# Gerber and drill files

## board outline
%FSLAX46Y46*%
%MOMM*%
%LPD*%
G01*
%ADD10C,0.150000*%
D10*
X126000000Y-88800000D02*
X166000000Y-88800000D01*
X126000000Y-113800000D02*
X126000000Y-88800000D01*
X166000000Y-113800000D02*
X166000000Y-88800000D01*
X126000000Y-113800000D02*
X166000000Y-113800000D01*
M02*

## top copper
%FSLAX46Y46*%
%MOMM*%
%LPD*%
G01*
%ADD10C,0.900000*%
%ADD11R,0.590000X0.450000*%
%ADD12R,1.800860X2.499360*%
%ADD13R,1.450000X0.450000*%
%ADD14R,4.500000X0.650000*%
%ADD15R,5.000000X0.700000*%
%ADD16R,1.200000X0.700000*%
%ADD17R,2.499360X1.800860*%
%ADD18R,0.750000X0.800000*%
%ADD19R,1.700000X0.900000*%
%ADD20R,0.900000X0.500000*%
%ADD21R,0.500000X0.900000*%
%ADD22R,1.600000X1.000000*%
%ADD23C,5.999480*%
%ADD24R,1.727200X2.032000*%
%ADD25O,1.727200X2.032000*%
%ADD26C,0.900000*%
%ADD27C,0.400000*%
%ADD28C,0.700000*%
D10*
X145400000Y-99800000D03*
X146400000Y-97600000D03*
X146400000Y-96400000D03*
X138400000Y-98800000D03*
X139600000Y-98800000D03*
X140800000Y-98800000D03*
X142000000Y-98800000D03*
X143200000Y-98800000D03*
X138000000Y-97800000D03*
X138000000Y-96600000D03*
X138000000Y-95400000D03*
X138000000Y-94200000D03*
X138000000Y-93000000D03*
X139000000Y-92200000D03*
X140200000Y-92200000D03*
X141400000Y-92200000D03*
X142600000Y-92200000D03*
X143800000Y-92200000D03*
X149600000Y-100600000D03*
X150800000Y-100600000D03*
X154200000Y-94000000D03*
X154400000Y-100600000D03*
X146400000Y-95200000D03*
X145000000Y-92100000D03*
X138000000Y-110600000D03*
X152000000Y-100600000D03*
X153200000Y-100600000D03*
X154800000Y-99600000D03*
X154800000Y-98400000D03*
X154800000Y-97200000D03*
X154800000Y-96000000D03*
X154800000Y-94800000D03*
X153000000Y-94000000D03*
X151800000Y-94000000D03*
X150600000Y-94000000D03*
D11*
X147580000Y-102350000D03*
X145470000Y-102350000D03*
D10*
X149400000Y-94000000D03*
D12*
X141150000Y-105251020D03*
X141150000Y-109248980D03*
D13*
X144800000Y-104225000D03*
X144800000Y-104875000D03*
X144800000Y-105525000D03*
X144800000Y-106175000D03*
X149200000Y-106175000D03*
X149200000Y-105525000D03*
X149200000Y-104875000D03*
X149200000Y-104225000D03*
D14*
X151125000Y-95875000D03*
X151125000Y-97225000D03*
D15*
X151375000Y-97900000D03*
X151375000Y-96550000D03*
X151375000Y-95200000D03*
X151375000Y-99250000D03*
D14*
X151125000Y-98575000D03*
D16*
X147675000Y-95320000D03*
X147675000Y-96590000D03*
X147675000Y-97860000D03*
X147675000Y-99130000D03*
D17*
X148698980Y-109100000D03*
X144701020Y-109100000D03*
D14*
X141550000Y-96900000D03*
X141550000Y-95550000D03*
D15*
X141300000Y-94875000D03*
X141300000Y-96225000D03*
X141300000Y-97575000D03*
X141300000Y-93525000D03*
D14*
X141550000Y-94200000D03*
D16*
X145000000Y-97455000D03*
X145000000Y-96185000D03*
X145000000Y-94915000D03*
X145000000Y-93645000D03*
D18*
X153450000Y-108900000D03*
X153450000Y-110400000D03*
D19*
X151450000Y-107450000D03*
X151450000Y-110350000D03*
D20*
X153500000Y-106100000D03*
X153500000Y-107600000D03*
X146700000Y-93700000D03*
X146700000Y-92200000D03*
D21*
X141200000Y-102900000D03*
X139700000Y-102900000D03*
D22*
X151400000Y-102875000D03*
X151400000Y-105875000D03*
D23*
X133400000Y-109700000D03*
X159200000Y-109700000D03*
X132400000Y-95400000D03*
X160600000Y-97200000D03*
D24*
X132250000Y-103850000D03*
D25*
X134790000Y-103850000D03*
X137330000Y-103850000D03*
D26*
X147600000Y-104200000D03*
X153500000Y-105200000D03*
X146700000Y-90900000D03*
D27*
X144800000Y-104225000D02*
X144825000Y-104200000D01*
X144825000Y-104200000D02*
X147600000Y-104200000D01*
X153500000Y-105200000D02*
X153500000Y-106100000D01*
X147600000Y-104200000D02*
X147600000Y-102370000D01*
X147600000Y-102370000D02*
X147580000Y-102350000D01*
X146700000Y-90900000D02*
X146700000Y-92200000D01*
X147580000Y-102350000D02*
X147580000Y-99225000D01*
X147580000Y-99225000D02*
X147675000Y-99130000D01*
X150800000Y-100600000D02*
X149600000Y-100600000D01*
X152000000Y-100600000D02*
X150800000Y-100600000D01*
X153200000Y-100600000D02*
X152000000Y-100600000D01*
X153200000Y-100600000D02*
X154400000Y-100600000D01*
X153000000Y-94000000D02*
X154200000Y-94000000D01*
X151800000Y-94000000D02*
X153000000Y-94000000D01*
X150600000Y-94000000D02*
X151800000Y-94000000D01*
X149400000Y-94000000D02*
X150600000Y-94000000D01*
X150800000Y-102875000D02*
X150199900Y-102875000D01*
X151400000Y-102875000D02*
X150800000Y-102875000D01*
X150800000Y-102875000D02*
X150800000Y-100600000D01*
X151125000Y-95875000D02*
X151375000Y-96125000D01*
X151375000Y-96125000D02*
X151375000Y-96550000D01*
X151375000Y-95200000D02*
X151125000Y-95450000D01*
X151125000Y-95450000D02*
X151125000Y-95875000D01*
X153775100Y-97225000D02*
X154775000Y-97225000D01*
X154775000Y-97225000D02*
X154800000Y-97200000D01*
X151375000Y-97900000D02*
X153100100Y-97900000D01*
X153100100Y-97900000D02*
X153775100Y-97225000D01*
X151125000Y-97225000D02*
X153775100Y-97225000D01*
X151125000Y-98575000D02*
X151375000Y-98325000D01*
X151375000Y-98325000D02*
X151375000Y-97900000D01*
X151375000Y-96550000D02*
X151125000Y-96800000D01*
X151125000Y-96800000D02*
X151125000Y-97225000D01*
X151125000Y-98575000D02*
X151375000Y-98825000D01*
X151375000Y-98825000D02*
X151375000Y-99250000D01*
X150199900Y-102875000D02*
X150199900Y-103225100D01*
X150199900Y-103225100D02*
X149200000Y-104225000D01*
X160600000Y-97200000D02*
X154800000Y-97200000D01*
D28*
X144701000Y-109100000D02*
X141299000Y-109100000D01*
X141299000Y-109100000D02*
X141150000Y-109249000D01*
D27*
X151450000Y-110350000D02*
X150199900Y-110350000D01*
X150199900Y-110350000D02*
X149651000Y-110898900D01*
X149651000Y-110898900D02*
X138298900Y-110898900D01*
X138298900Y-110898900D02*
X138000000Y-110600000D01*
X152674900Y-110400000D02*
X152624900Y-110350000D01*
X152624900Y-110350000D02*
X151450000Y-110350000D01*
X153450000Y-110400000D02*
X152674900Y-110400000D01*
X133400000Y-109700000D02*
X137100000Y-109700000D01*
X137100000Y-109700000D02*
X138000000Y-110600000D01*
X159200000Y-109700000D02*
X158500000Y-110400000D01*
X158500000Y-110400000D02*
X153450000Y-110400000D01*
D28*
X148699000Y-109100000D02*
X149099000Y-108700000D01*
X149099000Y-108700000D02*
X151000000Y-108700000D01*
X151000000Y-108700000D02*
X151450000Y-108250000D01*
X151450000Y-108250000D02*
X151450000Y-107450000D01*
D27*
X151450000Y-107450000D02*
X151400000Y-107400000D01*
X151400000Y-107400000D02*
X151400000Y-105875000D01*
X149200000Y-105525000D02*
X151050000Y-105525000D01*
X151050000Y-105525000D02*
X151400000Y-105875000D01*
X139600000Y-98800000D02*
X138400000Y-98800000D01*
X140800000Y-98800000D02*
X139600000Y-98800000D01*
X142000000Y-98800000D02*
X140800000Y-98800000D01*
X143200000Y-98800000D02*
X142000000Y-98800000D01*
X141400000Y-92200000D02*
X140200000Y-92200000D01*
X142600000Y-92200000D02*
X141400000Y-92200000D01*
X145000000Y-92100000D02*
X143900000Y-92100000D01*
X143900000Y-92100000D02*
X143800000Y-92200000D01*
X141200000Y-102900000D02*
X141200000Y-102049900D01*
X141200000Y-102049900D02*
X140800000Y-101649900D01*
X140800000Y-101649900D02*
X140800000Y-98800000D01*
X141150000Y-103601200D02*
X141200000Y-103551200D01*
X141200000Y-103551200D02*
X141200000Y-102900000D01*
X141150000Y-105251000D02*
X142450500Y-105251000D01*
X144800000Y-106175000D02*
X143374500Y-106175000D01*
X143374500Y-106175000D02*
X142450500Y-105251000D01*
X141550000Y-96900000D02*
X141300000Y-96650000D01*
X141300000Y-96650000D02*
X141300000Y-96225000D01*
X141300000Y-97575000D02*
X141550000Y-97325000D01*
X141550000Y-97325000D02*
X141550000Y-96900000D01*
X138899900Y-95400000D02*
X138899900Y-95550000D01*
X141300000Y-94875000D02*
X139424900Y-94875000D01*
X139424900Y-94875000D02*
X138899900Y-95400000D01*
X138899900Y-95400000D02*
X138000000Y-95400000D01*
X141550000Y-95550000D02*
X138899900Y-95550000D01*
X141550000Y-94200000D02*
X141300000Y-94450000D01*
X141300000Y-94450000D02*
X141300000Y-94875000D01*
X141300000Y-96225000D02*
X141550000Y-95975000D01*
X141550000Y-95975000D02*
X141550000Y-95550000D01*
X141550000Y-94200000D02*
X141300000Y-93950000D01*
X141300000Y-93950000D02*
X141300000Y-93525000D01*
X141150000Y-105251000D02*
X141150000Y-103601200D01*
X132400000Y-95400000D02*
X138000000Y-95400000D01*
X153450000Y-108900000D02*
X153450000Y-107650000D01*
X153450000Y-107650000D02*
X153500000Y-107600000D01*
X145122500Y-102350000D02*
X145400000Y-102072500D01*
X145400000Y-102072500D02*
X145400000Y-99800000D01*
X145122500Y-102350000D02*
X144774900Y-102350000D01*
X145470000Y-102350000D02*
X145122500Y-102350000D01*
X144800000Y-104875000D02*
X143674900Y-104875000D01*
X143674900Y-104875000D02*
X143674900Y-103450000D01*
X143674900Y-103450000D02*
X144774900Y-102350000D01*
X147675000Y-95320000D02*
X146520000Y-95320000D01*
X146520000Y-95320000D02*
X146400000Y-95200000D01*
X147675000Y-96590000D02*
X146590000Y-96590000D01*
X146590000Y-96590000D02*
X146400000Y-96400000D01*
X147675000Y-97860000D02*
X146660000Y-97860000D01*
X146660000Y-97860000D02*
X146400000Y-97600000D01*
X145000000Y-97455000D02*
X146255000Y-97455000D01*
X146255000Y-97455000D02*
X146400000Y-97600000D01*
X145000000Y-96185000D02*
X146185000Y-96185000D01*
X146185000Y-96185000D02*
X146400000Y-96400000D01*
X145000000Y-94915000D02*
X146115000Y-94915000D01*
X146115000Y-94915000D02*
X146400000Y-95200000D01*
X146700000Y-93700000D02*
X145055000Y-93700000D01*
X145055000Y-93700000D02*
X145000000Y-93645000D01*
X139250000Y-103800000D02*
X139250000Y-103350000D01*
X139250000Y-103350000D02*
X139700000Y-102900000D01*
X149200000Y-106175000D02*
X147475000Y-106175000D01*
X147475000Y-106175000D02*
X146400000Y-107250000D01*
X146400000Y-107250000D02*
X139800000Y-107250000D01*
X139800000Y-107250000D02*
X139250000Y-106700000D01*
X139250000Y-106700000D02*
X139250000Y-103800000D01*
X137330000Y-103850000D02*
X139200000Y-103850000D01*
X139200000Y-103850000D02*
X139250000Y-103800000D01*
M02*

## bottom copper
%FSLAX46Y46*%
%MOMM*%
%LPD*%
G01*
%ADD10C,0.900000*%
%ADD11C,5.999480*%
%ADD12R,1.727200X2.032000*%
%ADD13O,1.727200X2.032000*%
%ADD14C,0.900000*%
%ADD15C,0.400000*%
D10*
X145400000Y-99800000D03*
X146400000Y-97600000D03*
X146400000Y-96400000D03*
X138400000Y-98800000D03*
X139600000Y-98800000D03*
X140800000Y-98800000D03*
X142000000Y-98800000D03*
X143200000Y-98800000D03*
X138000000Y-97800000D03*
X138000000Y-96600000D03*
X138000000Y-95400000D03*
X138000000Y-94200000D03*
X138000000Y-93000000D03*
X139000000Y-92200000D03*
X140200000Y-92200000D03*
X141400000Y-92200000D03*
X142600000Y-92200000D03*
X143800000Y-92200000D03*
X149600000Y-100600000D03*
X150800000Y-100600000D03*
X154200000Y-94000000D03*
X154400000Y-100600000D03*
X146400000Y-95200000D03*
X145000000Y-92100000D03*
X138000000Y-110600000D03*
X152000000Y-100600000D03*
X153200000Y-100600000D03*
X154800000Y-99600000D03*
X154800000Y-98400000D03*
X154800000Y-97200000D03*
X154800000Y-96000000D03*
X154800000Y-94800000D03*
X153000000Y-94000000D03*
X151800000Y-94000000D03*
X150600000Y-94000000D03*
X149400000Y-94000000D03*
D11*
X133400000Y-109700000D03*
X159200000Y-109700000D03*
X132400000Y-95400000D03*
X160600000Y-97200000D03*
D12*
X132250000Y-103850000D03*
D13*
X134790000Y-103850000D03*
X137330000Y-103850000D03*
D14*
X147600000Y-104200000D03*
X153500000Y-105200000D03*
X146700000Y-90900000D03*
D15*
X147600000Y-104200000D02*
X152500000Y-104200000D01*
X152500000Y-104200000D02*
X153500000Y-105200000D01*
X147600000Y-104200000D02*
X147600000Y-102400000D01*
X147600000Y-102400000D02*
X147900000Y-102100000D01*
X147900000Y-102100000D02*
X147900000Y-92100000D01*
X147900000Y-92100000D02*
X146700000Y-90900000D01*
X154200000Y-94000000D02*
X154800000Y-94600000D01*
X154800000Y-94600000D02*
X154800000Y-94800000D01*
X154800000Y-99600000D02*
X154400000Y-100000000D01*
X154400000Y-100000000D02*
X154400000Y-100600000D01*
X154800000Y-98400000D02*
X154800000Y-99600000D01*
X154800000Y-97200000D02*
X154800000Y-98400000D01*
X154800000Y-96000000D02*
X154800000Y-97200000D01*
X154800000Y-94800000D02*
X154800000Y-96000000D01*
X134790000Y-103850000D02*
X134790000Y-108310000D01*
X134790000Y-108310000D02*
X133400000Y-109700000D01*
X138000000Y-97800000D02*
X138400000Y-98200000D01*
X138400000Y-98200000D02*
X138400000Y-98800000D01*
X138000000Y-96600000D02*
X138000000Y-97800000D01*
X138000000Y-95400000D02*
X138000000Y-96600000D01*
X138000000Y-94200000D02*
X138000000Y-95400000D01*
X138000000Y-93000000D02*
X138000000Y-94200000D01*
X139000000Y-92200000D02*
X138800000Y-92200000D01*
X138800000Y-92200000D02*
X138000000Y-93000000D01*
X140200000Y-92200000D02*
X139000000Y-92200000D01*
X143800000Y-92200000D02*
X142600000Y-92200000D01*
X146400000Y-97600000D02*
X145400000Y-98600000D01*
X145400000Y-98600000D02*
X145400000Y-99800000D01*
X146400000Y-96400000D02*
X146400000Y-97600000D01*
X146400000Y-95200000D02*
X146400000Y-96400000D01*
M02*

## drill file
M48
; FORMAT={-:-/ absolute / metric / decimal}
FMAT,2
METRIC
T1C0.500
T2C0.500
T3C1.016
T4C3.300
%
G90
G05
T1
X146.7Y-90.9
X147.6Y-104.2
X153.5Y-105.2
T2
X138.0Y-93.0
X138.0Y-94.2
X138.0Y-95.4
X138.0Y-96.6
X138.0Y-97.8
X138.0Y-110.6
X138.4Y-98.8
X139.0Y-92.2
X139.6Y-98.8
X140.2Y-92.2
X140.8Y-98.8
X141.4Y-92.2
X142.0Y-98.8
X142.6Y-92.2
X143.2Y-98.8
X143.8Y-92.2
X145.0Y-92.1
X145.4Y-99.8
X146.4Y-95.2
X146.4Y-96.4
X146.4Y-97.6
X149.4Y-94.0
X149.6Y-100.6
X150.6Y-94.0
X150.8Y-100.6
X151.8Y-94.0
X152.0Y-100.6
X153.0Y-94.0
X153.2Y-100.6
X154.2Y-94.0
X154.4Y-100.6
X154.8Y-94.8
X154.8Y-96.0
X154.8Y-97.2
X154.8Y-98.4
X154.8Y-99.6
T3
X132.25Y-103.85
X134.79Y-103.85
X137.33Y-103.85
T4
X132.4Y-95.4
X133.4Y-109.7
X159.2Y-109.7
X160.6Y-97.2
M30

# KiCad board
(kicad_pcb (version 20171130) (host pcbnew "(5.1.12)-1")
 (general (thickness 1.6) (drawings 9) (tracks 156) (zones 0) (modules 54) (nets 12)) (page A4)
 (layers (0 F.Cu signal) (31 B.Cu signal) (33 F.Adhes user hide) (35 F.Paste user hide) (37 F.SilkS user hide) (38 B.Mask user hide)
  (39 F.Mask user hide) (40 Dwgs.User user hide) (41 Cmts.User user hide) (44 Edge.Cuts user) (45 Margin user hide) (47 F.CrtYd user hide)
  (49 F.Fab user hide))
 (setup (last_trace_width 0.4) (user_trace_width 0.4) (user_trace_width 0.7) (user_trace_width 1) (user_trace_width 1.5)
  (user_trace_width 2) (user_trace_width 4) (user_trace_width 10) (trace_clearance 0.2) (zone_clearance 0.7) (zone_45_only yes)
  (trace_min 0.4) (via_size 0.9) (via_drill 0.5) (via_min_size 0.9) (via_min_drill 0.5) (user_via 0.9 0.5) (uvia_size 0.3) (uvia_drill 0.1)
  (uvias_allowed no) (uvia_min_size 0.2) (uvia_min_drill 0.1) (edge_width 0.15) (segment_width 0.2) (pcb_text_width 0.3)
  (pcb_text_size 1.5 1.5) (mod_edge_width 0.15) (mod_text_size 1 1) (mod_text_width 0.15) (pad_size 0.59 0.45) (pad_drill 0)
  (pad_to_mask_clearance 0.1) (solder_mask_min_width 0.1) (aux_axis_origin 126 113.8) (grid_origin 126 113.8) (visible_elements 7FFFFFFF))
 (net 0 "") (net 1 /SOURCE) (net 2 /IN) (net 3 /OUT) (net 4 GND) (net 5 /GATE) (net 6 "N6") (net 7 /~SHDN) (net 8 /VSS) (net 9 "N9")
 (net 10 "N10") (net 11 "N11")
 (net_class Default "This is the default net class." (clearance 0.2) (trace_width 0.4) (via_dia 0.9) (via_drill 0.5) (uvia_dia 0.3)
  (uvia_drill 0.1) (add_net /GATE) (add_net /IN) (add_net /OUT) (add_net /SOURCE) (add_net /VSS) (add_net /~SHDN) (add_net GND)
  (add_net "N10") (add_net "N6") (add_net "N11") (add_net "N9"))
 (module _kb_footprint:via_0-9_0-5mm (layer F.Cu) (at 145.4 99.8)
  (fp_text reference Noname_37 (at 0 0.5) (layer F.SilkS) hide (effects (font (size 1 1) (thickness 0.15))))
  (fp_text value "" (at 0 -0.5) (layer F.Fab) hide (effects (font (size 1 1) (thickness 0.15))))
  (pad 1 thru_hole circle (at 0 0) (size 0.9 0.9) (drill 0.5) (layers *.Cu) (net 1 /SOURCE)))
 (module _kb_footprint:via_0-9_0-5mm (layer F.Cu) (at 146.4 97.6)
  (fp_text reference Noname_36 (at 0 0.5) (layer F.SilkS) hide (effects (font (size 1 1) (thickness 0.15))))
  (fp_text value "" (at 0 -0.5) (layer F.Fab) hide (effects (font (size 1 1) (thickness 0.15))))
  (pad 1 thru_hole circle (at 0 0) (size 0.9 0.9) (drill 0.5) (layers *.Cu) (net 1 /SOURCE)))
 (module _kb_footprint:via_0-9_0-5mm (layer F.Cu) (at 146.4 96.4)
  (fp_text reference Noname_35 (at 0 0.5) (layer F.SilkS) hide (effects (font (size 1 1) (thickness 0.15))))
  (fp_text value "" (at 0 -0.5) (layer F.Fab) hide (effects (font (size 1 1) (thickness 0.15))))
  (pad 1 thru_hole circle (at 0 0) (size 0.9 0.9) (drill 0.5) (layers *.Cu) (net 1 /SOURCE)))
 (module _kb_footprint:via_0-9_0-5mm (layer F.Cu) (at 138.4 98.8)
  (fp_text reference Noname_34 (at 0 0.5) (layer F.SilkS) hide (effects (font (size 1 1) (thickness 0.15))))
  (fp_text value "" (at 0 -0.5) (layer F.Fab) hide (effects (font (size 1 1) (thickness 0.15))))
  (pad 1 thru_hole circle (at 0 0) (size 0.9 0.9) (drill 0.5) (layers *.Cu) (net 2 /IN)))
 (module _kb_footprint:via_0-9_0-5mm (layer F.Cu) (at 139.6 98.8)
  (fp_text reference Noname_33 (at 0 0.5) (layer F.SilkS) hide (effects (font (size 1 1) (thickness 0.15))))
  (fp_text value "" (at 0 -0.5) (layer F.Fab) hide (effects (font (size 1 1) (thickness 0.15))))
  (pad 1 thru_hole circle (at 0 0) (size 0.9 0.9) (drill 0.5) (layers *.Cu) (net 2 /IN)))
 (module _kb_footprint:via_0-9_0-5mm (layer F.Cu) (at 140.8 98.8)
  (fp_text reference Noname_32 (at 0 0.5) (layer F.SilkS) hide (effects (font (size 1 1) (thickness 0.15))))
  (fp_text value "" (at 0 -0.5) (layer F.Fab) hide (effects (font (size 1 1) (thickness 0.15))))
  (pad 1 thru_hole circle (at 0 0) (size 0.9 0.9) (drill 0.5) (layers *.Cu) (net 2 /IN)))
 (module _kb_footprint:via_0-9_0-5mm (layer F.Cu) (at 142 98.8)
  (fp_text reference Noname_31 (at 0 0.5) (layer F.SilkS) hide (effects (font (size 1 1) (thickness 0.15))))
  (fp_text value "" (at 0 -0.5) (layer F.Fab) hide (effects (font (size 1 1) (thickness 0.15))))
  (pad 1 thru_hole circle (at 0 0) (size 0.9 0.9) (drill 0.5) (layers *.Cu) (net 2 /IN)))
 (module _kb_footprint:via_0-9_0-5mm (layer F.Cu) (at 143.2 98.8)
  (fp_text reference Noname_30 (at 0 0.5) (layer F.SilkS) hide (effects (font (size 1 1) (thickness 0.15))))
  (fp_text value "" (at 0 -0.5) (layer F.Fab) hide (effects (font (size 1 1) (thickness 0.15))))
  (pad 1 thru_hole circle (at 0 0) (size 0.9 0.9) (drill 0.5) (layers *.Cu) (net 2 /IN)))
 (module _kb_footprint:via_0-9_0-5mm (layer F.Cu) (at 138 97.8)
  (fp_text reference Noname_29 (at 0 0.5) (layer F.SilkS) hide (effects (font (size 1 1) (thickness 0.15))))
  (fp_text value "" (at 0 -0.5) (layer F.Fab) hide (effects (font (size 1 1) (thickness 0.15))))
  (pad 1 thru_hole circle (at 0 0) (size 0.9 0.9) (drill 0.5) (layers *.Cu) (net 2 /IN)))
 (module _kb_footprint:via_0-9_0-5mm (layer F.Cu) (at 138 96.6)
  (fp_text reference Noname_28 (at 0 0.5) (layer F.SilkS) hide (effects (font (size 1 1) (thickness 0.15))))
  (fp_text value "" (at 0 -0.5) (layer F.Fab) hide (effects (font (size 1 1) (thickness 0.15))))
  (pad 1 thru_hole circle (at 0 0) (size 0.9 0.9) (drill 0.5) (layers *.Cu) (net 2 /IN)))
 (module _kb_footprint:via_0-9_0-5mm (layer F.Cu) (at 138 95.4)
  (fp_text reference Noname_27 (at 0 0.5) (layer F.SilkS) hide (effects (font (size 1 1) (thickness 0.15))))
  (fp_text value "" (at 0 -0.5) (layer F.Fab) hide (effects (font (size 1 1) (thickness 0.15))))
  (pad 1 thru_hole circle (at 0 0) (size 0.9 0.9) (drill 0.5) (layers *.Cu) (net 2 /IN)))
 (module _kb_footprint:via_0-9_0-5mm (layer F.Cu) (at 138 94.2)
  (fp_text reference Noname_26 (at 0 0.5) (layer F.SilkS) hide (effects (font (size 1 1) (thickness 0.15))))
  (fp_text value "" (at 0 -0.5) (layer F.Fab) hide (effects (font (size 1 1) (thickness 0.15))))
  (pad 1 thru_hole circle (at 0 0) (size 0.9 0.9) (drill 0.5) (layers *.Cu) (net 2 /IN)))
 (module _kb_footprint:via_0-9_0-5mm (layer F.Cu) (at 138 93)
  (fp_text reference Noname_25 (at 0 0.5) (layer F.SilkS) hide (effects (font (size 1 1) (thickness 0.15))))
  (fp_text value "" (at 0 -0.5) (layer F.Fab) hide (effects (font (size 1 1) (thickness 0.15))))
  (pad 1 thru_hole circle (at 0 0) (size 0.9 0.9) (drill 0.5) (layers *.Cu) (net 2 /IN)))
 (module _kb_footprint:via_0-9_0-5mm (layer F.Cu) (at 139 92.2)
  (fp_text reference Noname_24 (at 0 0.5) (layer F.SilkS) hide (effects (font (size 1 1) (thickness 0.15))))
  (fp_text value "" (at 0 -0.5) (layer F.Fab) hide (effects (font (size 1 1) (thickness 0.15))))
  (pad 1 thru_hole circle (at 0 0) (size 0.9 0.9) (drill 0.5) (layers *.Cu) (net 2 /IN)))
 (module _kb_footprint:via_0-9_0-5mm (layer F.Cu) (at 140.2 92.2)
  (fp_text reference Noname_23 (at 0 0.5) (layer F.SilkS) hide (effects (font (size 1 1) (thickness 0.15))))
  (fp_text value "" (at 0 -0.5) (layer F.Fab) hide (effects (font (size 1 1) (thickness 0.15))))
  (pad 1 thru_hole circle (at 0 0) (size 0.9 0.9) (drill 0.5) (layers *.Cu) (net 2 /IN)))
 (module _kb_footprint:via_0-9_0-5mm (layer F.Cu) (at 141.4 92.2)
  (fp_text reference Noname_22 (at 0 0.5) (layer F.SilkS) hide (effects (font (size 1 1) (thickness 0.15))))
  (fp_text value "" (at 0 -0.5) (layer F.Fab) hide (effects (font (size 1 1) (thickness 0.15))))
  (pad 1 thru_hole circle (at 0 0) (size 0.9 0.9) (drill 0.5) (layers *.Cu) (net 2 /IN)))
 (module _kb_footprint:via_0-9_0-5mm (layer F.Cu) (at 142.6 92.2)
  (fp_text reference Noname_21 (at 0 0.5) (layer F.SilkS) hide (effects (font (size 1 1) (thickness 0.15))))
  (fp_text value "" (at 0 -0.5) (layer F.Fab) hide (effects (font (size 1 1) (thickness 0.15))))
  (pad 1 thru_hole circle (at 0 0) (size 0.9 0.9) (drill 0.5) (layers *.Cu) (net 2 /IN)))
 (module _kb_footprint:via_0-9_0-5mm (layer F.Cu) (at 143.8 92.2)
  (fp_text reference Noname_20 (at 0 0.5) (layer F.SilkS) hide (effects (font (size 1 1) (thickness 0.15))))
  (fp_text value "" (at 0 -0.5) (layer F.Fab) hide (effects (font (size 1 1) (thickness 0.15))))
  (pad 1 thru_hole circle (at 0 0) (size 0.9 0.9) (drill 0.5) (layers *.Cu) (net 2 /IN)))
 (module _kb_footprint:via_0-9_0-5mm (layer F.Cu) (at 149.6 100.6)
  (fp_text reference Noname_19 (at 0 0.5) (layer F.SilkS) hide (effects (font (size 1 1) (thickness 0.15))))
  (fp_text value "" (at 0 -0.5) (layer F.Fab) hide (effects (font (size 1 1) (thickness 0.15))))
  (pad 1 thru_hole circle (at 0 0) (size 0.9 0.9) (drill 0.5) (layers *.Cu) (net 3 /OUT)))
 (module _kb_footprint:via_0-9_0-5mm (layer F.Cu) (at 150.8 100.6)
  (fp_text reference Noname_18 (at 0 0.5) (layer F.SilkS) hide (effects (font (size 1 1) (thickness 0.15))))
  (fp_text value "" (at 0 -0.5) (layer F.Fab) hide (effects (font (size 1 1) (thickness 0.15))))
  (pad 1 thru_hole circle (at 0 0) (size 0.9 0.9) (drill 0.5) (layers *.Cu) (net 3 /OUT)))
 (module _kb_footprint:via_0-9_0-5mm (layer F.Cu) (at 154.2 94)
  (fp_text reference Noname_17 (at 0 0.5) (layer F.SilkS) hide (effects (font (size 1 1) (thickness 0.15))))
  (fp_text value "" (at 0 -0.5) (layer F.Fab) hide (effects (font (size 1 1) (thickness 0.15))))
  (pad 1 thru_hole circle (at 0 0) (size 0.9 0.9) (drill 0.5) (layers *.Cu) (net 3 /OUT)))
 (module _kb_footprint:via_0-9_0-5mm (layer F.Cu) (at 154.4 100.6)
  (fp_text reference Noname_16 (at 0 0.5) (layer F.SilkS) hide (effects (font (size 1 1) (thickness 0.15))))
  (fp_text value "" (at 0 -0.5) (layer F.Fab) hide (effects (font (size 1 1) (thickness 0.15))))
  (pad 1 thru_hole circle (at 0 0) (size 0.9 0.9) (drill 0.5) (layers *.Cu) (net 3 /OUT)))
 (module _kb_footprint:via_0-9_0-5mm (layer F.Cu) (at 146.4 95.2)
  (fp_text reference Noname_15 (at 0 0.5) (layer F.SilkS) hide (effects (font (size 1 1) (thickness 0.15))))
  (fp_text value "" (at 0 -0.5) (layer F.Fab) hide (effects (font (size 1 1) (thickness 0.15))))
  (pad 1 thru_hole circle (at 0 0) (size 0.9 0.9) (drill 0.5) (layers *.Cu) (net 1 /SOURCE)))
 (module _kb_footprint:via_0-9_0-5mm (layer F.Cu) (at 145 92.1)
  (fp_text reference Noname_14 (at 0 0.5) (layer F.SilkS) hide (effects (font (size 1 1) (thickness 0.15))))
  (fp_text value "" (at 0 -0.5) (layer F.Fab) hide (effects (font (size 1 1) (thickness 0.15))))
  (pad 1 thru_hole circle (at 0 0) (size 0.9 0.9) (drill 0.5) (layers *.Cu) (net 2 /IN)))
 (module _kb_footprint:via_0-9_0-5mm (layer F.Cu) (at 138 110.6)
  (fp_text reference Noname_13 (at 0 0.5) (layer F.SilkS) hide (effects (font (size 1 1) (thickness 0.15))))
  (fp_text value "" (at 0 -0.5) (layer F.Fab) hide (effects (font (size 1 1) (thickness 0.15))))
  (pad 1 thru_hole circle (at 0 0) (size 0.9 0.9) (drill 0.5) (layers *.Cu) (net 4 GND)))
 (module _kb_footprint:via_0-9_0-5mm (layer F.Cu) (at 152 100.6)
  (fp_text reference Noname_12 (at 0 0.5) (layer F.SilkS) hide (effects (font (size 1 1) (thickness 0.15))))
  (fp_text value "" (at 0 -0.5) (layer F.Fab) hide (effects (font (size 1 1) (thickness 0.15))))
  (pad 1 thru_hole circle (at 0 0) (size 0.9 0.9) (drill 0.5) (layers *.Cu) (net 3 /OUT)))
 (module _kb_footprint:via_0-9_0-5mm (layer F.Cu) (at 153.2 100.6)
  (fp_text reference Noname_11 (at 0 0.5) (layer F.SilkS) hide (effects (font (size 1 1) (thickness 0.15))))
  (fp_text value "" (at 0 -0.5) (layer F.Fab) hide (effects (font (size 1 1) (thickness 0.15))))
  (pad 1 thru_hole circle (at 0 0) (size 0.9 0.9) (drill 0.5) (layers *.Cu) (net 3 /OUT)))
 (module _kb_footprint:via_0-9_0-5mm (layer F.Cu) (at 154.8 99.6)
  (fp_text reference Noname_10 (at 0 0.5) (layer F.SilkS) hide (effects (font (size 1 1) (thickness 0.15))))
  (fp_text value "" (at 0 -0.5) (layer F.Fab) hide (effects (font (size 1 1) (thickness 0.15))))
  (pad 1 thru_hole circle (at 0 0) (size 0.9 0.9) (drill 0.5) (layers *.Cu) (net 3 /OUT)))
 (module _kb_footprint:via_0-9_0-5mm (layer F.Cu) (at 154.8 98.4)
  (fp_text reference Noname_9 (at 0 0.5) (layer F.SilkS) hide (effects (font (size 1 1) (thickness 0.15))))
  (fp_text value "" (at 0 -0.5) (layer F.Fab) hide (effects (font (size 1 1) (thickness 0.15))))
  (pad 1 thru_hole circle (at 0 0) (size 0.9 0.9) (drill 0.5) (layers *.Cu) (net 3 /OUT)))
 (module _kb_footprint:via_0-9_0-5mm (layer F.Cu) (at 154.8 97.2)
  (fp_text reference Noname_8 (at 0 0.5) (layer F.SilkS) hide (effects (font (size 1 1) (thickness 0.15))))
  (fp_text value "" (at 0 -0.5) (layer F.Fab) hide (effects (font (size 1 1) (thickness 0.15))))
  (pad 1 thru_hole circle (at 0 0) (size 0.9 0.9) (drill 0.5) (layers *.Cu) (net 3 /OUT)))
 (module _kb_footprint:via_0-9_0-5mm (layer F.Cu) (at 154.8 96)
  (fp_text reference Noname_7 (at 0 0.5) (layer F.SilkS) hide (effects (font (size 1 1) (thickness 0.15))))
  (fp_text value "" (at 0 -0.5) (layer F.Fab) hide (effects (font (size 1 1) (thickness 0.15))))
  (pad 1 thru_hole circle (at 0 0) (size 0.9 0.9) (drill 0.5) (layers *.Cu) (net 3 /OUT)))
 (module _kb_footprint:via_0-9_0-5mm (layer F.Cu) (at 154.8 94.8)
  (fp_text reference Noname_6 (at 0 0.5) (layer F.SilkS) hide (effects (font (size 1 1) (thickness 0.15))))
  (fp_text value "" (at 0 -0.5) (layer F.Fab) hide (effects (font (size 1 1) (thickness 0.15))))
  (pad 1 thru_hole circle (at 0 0) (size 0.9 0.9) (drill 0.5) (layers *.Cu) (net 3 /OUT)))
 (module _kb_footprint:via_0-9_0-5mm (layer F.Cu) (at 153 94)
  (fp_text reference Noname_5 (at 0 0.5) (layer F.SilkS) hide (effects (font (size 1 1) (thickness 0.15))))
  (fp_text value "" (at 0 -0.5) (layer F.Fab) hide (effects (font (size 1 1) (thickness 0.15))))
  (pad 1 thru_hole circle (at 0 0) (size 0.9 0.9) (drill 0.5) (layers *.Cu) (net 3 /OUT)))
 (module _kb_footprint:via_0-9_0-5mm (layer F.Cu) (at 151.8 94)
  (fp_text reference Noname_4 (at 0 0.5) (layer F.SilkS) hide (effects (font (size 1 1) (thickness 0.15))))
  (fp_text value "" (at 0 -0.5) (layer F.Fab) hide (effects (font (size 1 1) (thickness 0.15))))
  (pad 1 thru_hole circle (at 0 0) (size 0.9 0.9) (drill 0.5) (layers *.Cu) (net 3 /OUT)))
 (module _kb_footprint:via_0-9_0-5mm (layer F.Cu) (at 150.6 94)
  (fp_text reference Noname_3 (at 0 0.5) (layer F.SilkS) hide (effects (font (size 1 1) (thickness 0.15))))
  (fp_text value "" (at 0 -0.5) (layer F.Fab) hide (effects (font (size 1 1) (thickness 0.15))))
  (pad 1 thru_hole circle (at 0 0) (size 0.9 0.9) (drill 0.5) (layers *.Cu) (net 3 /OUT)))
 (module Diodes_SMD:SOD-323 (layer F.Cu) (at 146.525 102.35 180)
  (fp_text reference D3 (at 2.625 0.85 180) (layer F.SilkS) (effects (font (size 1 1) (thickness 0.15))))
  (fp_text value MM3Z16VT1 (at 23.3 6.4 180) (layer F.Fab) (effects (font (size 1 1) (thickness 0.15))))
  (pad 1 smd rect (at -1.055 0 180) (size 0.59 0.45) (layers F.Cu F.Paste F.Mask) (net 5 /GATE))
  (pad 2 smd rect (at 1.055 0 180) (size 0.59 0.45) (layers F.Cu F.Paste F.Mask) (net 1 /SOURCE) (zone_connect 1)))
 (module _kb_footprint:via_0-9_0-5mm (layer F.Cu) (at 149.4 94)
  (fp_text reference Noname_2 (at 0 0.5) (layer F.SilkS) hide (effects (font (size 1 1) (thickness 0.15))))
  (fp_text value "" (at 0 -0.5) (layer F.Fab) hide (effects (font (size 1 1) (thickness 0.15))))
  (pad 1 thru_hole circle (at 0 0) (size 0.9 0.9) (drill 0.5) (layers *.Cu) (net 3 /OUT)))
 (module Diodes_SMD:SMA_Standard (layer F.Cu) (at 141.15 107.25 270)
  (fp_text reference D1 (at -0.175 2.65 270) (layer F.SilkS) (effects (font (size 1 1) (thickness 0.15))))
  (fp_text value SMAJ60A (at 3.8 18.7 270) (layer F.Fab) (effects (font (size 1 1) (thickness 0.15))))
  (pad 1 smd rect (at -1.99898 0 270) (size 2.49936 1.80086) (layers F.Cu F.Paste F.Mask) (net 2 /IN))
  (pad 2 smd rect (at 1.99898 0 270) (size 2.49936 1.80086) (layers F.Cu F.Paste F.Mask) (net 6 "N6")))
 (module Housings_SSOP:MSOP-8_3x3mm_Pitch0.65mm (layer F.Cu) (at 147 105.2)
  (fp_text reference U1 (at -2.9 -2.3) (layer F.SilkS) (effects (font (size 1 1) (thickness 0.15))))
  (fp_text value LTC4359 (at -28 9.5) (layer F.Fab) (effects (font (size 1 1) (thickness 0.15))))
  (pad 1 smd rect (at -2.2 -0.975) (size 1.45 0.45) (layers F.Cu F.Paste F.Mask) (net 5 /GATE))
  (pad 2 smd rect (at -2.2 -0.325) (size 1.45 0.45) (layers F.Cu F.Paste F.Mask) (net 1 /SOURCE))
  (pad 3 smd rect (at -2.2 0.325) (size 1.45 0.45) (layers F.Cu F.Paste F.Mask))
  (pad 4 smd rect (at -2.2 0.975) (size 1.45 0.45) (layers F.Cu F.Paste F.Mask) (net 2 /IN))
  (pad 5 smd rect (at 2.2 0.975) (size 1.45 0.45) (layers F.Cu F.Paste F.Mask) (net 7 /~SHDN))
  (pad 6 smd rect (at 2.2 0.325) (size 1.45 0.45) (layers F.Cu F.Paste F.Mask) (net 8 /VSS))
  (pad 7 smd rect (at 2.2 -0.325) (size 1.45 0.45) (layers F.Cu F.Paste F.Mask))
  (pad 8 smd rect (at 2.2 -0.975) (size 1.45 0.45) (layers F.Cu F.Paste F.Mask) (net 3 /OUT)))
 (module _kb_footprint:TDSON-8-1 (layer F.Cu) (at 150.475 97.225)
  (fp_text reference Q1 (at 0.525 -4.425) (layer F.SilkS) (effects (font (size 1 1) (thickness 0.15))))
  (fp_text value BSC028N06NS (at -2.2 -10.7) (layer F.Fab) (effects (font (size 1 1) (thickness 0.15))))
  (pad 7 smd rect (at 0.65 -1.35) (size 4.5 0.65) (layers F.Cu F.Paste F.Mask) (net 3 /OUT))
  (pad 6 smd rect (at 0.65 0) (size 4.5 0.65) (layers F.Cu F.Paste F.Mask) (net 3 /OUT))
  (pad 6 smd rect (at 0.9 0.675) (size 5 0.7) (layers F.Cu F.Paste F.Mask) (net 3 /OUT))
  (pad 7 smd rect (at 0.9 -0.675) (size 5 0.7) (layers F.Cu F.Paste F.Mask) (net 3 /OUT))
  (pad 8 smd rect (at 0.9 -2.025) (size 5 0.7) (layers F.Cu F.Paste F.Mask) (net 3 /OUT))
  (pad 5 smd rect (at 0.9 2.025) (size 5 0.7) (layers F.Cu F.Paste F.Mask) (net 3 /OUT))
  (pad 5 smd rect (at 0.65 1.35) (size 4.5 0.65) (layers F.Cu F.Paste F.Mask) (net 3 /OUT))
  (pad 1 smd rect (at -2.8 -1.905) (size 1.2 0.7) (layers F.Cu F.Paste F.Mask) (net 1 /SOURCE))
  (pad 2 smd rect (at -2.8 -0.635) (size 1.2 0.7) (layers F.Cu F.Paste F.Mask) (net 1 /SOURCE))
  (pad 3 smd rect (at -2.8 0.635) (size 1.2 0.7) (layers F.Cu F.Paste F.Mask) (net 1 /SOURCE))
  (pad 4 smd rect (at -2.8 1.905) (size 1.2 0.7) (layers F.Cu F.Paste F.Mask) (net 5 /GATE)))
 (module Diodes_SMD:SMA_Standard (layer F.Cu) (at 146.7 109.1 180)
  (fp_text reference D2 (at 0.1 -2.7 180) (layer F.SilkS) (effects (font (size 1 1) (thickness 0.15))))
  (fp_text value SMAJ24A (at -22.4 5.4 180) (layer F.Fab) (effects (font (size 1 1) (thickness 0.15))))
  (pad 1 smd rect (at -1.99898 0 180) (size 2.49936 1.80086) (layers F.Cu F.Paste F.Mask) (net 8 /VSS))
  (pad 2 smd rect (at 1.99898 0 180) (size 2.49936 1.80086) (layers F.Cu F.Paste F.Mask) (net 6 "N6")))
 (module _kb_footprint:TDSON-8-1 (layer F.Cu) (at 142.2 95.55 180)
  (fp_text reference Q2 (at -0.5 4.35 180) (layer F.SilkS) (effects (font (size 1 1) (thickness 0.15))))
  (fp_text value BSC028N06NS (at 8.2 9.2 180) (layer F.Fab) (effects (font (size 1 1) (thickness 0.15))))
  (pad 7 smd rect (at 0.65 -1.35 180) (size 4.5 0.65) (layers F.Cu F.Paste F.Mask) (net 2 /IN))
  (pad 6 smd rect (at 0.65 0 180) (size 4.5 0.65) (layers F.Cu F.Paste F.Mask) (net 2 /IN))
  (pad 6 smd rect (at 0.9 0.675 180) (size 5 0.7) (layers F.Cu F.Paste F.Mask) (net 2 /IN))
  (pad 7 smd rect (at 0.9 -0.675 180) (size 5 0.7) (layers F.Cu F.Paste F.Mask) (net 2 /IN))
  (pad 8 smd rect (at 0.9 -2.025 180) (size 5 0.7) (layers F.Cu F.Paste F.Mask) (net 2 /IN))
  (pad 5 smd rect (at 0.9 2.025 180) (size 5 0.7) (layers F.Cu F.Paste F.Mask) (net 2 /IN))
  (pad 5 smd rect (at 0.65 1.35 180) (size 4.5 0.65) (layers F.Cu F.Paste F.Mask) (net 2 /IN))
  (pad 1 smd rect (at -2.8 -1.905 180) (size 1.2 0.7) (layers F.Cu F.Paste F.Mask) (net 1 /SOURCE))
  (pad 2 smd rect (at -2.8 -0.635 180) (size 1.2 0.7) (layers F.Cu F.Paste F.Mask) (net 1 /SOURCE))
  (pad 3 smd rect (at -2.8 0.635 180) (size 1.2 0.7) (layers F.Cu F.Paste F.Mask) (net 1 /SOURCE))
  (pad 4 smd rect (at -2.8 1.905 180) (size 1.2 0.7) (layers F.Cu F.Paste F.Mask) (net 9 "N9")))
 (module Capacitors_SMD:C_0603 (layer F.Cu) (at 153.45 109.65 270)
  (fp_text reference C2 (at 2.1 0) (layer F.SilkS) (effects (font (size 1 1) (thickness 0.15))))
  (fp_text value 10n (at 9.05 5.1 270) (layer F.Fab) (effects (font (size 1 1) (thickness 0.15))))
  (pad 1 smd rect (at -0.75 0 270) (size 0.8 0.75) (layers F.Cu F.Paste F.Mask) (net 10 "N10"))
  (pad 2 smd rect (at 0.75 0 270) (size 0.8 0.75) (layers F.Cu F.Paste F.Mask) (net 4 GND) (zone_connect 1)))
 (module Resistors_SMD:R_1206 (layer F.Cu) (at 151.45 108.9 270)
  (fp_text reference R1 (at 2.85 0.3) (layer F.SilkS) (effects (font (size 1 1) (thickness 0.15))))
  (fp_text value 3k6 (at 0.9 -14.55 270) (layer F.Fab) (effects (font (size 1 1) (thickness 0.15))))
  (pad 1 smd rect (at -1.45 0 270) (size 0.9 1.7) (layers F.Cu F.Paste F.Mask) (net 8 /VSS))
  (pad 2 smd rect (at 1.45 0 270) (size 0.9 1.7) (layers F.Cu F.Paste F.Mask) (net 4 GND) (zone_connect 1)))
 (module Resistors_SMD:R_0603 (layer F.Cu) (at 153.5 106.85 270)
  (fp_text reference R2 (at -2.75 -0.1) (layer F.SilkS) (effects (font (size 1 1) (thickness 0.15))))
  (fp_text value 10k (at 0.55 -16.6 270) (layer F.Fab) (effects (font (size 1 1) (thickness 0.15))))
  (pad 1 smd rect (at -0.75 0 270) (size 0.5 0.9) (layers F.Cu F.Paste F.Mask) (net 5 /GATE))
  (pad 2 smd rect (at 0.75 0 270) (size 0.5 0.9) (layers F.Cu F.Paste F.Mask) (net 10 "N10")))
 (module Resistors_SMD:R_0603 (layer F.Cu) (at 146.7 92.95 90)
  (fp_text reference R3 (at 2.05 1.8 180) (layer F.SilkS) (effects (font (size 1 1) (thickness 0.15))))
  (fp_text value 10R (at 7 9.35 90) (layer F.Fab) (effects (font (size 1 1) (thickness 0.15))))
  (pad 1 smd rect (at -0.75 0 90) (size 0.5 0.9) (layers F.Cu F.Paste F.Mask) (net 9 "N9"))
  (pad 2 smd rect (at 0.75 0 90) (size 0.5 0.9) (layers F.Cu F.Paste F.Mask) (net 5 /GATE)))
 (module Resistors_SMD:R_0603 (layer F.Cu) (at 140.45 102.9 180)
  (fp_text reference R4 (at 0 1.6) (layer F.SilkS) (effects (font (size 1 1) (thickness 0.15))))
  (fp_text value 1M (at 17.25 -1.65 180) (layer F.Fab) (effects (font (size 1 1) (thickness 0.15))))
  (pad 1 smd rect (at -0.75 0 180) (size 0.5 0.9) (layers F.Cu F.Paste F.Mask) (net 2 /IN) (zone_connect 1))
  (pad 2 smd rect (at 0.75 0 180) (size 0.5 0.9) (layers F.Cu F.Paste F.Mask) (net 7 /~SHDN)))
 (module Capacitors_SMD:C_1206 (layer F.Cu) (at 151.4 104.375 270)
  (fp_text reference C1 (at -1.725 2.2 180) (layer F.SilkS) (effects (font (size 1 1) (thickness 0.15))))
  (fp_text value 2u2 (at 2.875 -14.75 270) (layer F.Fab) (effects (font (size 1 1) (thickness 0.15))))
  (pad 1 smd rect (at -1.5 0 270) (size 1 1.6) (layers F.Cu F.Paste F.Mask) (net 3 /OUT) (zone_connect 1))
  (pad 2 smd rect (at 1.5 0 270) (size 1 1.6) (layers F.Cu F.Paste F.Mask) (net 8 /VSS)))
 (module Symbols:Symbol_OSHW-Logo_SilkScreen (layer F.Cu) (at 174 87)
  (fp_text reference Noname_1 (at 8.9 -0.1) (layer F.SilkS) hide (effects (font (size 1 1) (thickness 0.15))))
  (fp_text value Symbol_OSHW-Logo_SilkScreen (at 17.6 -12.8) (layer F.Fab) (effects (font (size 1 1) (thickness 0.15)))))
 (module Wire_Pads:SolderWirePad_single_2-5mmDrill (layer F.Cu) (at 133.4 109.7)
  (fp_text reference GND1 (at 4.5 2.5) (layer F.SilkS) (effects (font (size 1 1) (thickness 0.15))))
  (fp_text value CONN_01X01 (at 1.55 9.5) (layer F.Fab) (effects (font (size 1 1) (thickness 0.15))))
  (pad 1 thru_hole circle (at 0 0) (size 5.99948 5.99948) (drill 3.3) (layers *.Cu *.Mask F.SilkS) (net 4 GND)))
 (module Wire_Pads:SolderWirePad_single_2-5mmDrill (layer F.Cu) (at 159.2 109.7)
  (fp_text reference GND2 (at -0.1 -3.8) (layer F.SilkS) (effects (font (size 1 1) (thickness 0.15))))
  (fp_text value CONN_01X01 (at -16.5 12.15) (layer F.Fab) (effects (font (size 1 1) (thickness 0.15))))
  (pad 1 thru_hole circle (at 0 0) (size 5.99948 5.99948) (drill 3.3) (layers *.Cu *.Mask F.SilkS) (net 4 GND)))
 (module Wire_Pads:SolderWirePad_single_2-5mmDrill (layer F.Cu) (at 132.4 95.4)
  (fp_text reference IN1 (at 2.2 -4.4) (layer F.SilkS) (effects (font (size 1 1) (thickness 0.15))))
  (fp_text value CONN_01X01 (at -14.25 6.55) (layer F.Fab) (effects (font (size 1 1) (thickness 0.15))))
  (pad 1 thru_hole circle (at 0 0) (size 5.99948 5.99948) (drill 3.3) (layers *.Cu *.Mask F.SilkS) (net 2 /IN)))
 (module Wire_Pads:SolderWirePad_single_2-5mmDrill (layer F.Cu) (at 160.6 97.2)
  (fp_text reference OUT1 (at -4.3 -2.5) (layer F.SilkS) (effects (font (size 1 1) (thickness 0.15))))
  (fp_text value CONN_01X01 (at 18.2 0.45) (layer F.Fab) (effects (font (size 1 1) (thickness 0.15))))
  (pad 1 thru_hole circle (at 0 0) (size 5.99948 5.99948) (drill 3.3) (layers *.Cu *.Mask F.SilkS) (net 3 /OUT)))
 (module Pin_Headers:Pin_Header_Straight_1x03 (layer F.Cu) (at 132.25 103.85 90)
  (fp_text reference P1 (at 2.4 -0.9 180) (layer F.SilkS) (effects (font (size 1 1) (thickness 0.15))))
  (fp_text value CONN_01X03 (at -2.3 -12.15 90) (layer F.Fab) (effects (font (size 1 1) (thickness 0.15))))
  (pad 1 thru_hole rect (at 0 0 90) (size 2.032 1.7272) (drill 1.016) (layers *.Cu *.Mask F.SilkS) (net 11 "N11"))
  (pad 2 thru_hole oval (at 0 2.54 90) (size 2.032 1.7272) (drill 1.016) (layers *.Cu *.Mask F.SilkS) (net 4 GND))
  (pad 3 thru_hole oval (at 0 5.08 90) (size 2.032 1.7272) (drill 1.016) (layers *.Cu *.Mask F.SilkS) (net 7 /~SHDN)))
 (gr_line (start 126 88.8) (end 166 88.8) (angle 90) (layer Edge.Cuts) (width 0.15))
 (gr_line (start 126 113.8) (end 126 88.8) (angle 90) (layer Edge.Cuts) (width 0.15))
 (gr_line (start 166 113.8) (end 166 88.8) (angle 90) (layer Edge.Cuts) (width 0.15))
 (gr_line (start 126 113.8) (end 166 113.8) (angle 90) (layer Edge.Cuts) (width 0.15))
 (segment (start 144.8 104.225) (end 144.825 104.2) (width 0.4) (layer F.Cu) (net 5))
 (segment (start 144.825 104.2) (end 147.6 104.2) (width 0.4) (layer F.Cu) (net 5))
 (segment (start 147.6 104.2) (end 152.5 104.2) (width 0.4) (layer B.Cu) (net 5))
 (segment (start 152.5 104.2) (end 153.5 105.2) (width 0.4) (layer B.Cu) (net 5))
 (segment (start 153.5 105.2) (end 153.5 106.1) (width 0.4) (layer F.Cu) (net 5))
 (segment (start 147.6 104.2) (end 147.6 102.37) (width 0.4) (layer F.Cu) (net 5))
 (segment (start 147.6 102.37) (end 147.58 102.35) (width 0.4) (layer F.Cu) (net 5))
 (segment (start 146.7 90.9) (end 146.7 92.2) (width 0.4) (layer F.Cu) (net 5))
 (segment (start 147.6 104.2) (end 147.6 102.4) (width 0.4) (layer B.Cu) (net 5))
 (segment (start 147.6 102.4) (end 147.9 102.1) (width 0.4) (layer B.Cu) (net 5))
 (segment (start 147.9 102.1) (end 147.9 92.1) (width 0.4) (layer B.Cu) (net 5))
 (segment (start 147.9 92.1) (end 146.7 90.9) (width 0.4) (layer B.Cu) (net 5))
 (segment (start 147.58 102.35) (end 147.58 99.225) (width 0.4) (layer F.Cu) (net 5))
 (segment (start 147.58 99.225) (end 147.675 99.13) (width 0.4) (layer F.Cu) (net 5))
 (via (at 147.6 104.2) (size 0.9) (layers F.Cu B.Cu) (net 5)) (via (at 153.5 105.2) (size 0.9) (layers F.Cu B.Cu) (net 5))
 (via (at 146.7 90.9) (size 0.9) (layers F.Cu B.Cu) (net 5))
 (segment (start 150.8 100.6) (end 149.6 100.6) (width 0.4) (layer F.Cu) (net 3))
 (segment (start 152 100.6) (end 150.8 100.6) (width 0.4) (layer F.Cu) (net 3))
 (segment (start 154.2 94) (end 154.8 94.6) (width 0.4) (layer B.Cu) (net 3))
 (segment (start 154.8 94.6) (end 154.8 94.8) (width 0.4) (layer B.Cu) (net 3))
 (segment (start 153.2 100.6) (end 152 100.6) (width 0.4) (layer F.Cu) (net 3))
 (segment (start 153.2 100.6) (end 154.4 100.6) (width 0.4) (layer F.Cu) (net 3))
 (segment (start 154.8 99.6) (end 154.4 100) (width 0.4) (layer B.Cu) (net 3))
 (segment (start 154.4 100) (end 154.4 100.6) (width 0.4) (layer B.Cu) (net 3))
 (segment (start 154.8 98.4) (end 154.8 99.6) (width 0.4) (layer B.Cu) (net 3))
 (segment (start 154.8 97.2) (end 154.8 98.4) (width 0.4) (layer B.Cu) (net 3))
 (segment (start 154.8 96) (end 154.8 97.2) (width 0.4) (layer B.Cu) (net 3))
 (segment (start 154.8 94.8) (end 154.8 96) (width 0.4) (layer B.Cu) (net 3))
 (segment (start 153 94) (end 154.2 94) (width 0.4) (layer F.Cu) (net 3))
 (segment (start 151.8 94) (end 153 94) (width 0.4) (layer F.Cu) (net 3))
 (segment (start 150.6 94) (end 151.8 94) (width 0.4) (layer F.Cu) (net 3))
 (segment (start 149.4 94) (end 150.6 94) (width 0.4) (layer F.Cu) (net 3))
 (segment (start 150.8 102.875) (end 150.1999 102.875) (width 0.4) (layer F.Cu) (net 3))
 (segment (start 151.4 102.875) (end 150.8 102.875) (width 0.4) (layer F.Cu) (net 3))
 (segment (start 150.8 102.875) (end 150.8 100.6) (width 0.4) (layer F.Cu) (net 3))
 (segment (start 151.125 95.875) (end 151.375 96.125) (width 0.4) (layer F.Cu) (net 3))
 (segment (start 151.375 96.125) (end 151.375 96.55) (width 0.4) (layer F.Cu) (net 3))
 (segment (start 151.375 95.2) (end 151.125 95.45) (width 0.4) (layer F.Cu) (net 3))
 (segment (start 151.125 95.45) (end 151.125 95.875) (width 0.4) (layer F.Cu) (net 3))
 (segment (start 153.7751 97.225) (end 154.775 97.225) (width 0.4) (layer F.Cu) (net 3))
 (segment (start 154.775 97.225) (end 154.8 97.2) (width 0.4) (layer F.Cu) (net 3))
 (segment (start 151.375 97.9) (end 153.1001 97.9) (width 0.4) (layer F.Cu) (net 3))
 (segment (start 153.1001 97.9) (end 153.7751 97.225) (width 0.4) (layer F.Cu) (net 3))
 (segment (start 151.125 97.225) (end 153.7751 97.225) (width 0.4) (layer F.Cu) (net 3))
 (segment (start 151.125 98.575) (end 151.375 98.325) (width 0.4) (layer F.Cu) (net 3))
 (segment (start 151.375 98.325) (end 151.375 97.9) (width 0.4) (layer F.Cu) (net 3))
 (segment (start 151.375 96.55) (end 151.125 96.8) (width 0.4) (layer F.Cu) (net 3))
 (segment (start 151.125 96.8) (end 151.125 97.225) (width 0.4) (layer F.Cu) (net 3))
 (segment (start 151.125 98.575) (end 151.375 98.825) (width 0.4) (layer F.Cu) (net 3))
 (segment (start 151.375 98.825) (end 151.375 99.25) (width 0.4) (layer F.Cu) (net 3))
 (segment (start 150.1999 102.875) (end 150.1999 103.2251) (width 0.4) (layer F.Cu) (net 3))
 (segment (start 150.1999 103.2251) (end 149.2 104.225) (width 0.4) (layer F.Cu) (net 3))
 (segment (start 160.6 97.2) (end 154.8 97.2) (width 0.4) (layer F.Cu) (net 3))
 (segment (start 144.701 109.1) (end 141.299 109.1) (width 0.7) (layer F.Cu) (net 6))
 (segment (start 141.299 109.1) (end 141.15 109.249) (width 0.7) (layer F.Cu) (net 6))
 (segment (start 151.45 110.35) (end 150.1999 110.35) (width 0.4) (layer F.Cu) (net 4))
 (segment (start 150.1999 110.35) (end 149.651 110.8989) (width 0.4) (layer F.Cu) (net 4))
 (segment (start 149.651 110.8989) (end 138.2989 110.8989) (width 0.4) (layer F.Cu) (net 4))
 (segment (start 138.2989 110.8989) (end 138 110.6) (width 0.4) (layer F.Cu) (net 4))
 (segment (start 152.6749 110.4) (end 152.6249 110.35) (width 0.4) (layer F.Cu) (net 4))
 (segment (start 152.6249 110.35) (end 151.45 110.35) (width 0.4) (layer F.Cu) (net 4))
 (segment (start 153.45 110.4) (end 152.6749 110.4) (width 0.4) (layer F.Cu) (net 4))
 (segment (start 133.4 109.7) (end 137.1 109.7) (width 0.4) (layer F.Cu) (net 4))
 (segment (start 137.1 109.7) (end 138 110.6) (width 0.4) (layer F.Cu) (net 4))
 (segment (start 159.2 109.7) (end 158.5 110.4) (width 0.4) (layer F.Cu) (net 4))
 (segment (start 158.5 110.4) (end 153.45 110.4) (width 0.4) (layer F.Cu) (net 4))
 (segment (start 134.79 103.85) (end 134.79 108.31) (width 0.4) (layer B.Cu) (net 4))
 (segment (start 134.79 108.31) (end 133.4 109.7) (width 0.4) (layer B.Cu) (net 4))
 (segment (start 148.699 109.1) (end 149.099 108.7) (width 0.7) (layer F.Cu) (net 8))
 (segment (start 149.099 108.7) (end 151 108.7) (width 0.7) (layer F.Cu) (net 8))
 (segment (start 151 108.7) (end 151.45 108.25) (width 0.7) (layer F.Cu) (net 8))
 (segment (start 151.45 108.25) (end 151.45 107.45) (width 0.7) (layer F.Cu) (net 8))
 (segment (start 151.45 107.45) (end 151.4 107.4) (width 0.4) (layer F.Cu) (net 8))
 (segment (start 151.4 107.4) (end 151.4 105.875) (width 0.4) (layer F.Cu) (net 8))
 (segment (start 149.2 105.525) (end 151.05 105.525) (width 0.4) (layer F.Cu) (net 8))
 (segment (start 151.05 105.525) (end 151.4 105.875) (width 0.4) (layer F.Cu) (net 8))
 (segment (start 139.6 98.8) (end 138.4 98.8) (width 0.4) (layer F.Cu) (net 2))
 (segment (start 140.8 98.8) (end 139.6 98.8) (width 0.4) (layer F.Cu) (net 2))
 (segment (start 142 98.8) (end 140.8 98.8) (width 0.4) (layer F.Cu) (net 2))
 (segment (start 143.2 98.8) (end 142 98.8) (width 0.4) (layer F.Cu) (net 2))
 (segment (start 138 97.8) (end 138.4 98.2) (width 0.4) (layer B.Cu) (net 2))
 (segment (start 138.4 98.2) (end 138.4 98.8) (width 0.4) (layer B.Cu) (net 2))
 (segment (start 138 96.6) (end 138 97.8) (width 0.4) (layer B.Cu) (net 2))
 (segment (start 138 95.4) (end 138 96.6) (width 0.4) (layer B.Cu) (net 2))
 (segment (start 138 94.2) (end 138 95.4) (width 0.4) (layer B.Cu) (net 2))
 (segment (start 138 93) (end 138 94.2) (width 0.4) (layer B.Cu) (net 2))
 (segment (start 139 92.2) (end 138.8 92.2) (width 0.4) (layer B.Cu) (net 2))
 (segment (start 138.8 92.2) (end 138 93) (width 0.4) (layer B.Cu) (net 2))
 (segment (start 140.2 92.2) (end 139 92.2) (width 0.4) (layer B.Cu) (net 2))
 (segment (start 141.4 92.2) (end 140.2 92.2) (width 0.4) (layer F.Cu) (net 2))
 (segment (start 142.6 92.2) (end 141.4 92.2) (width 0.4) (layer F.Cu) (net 2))
 (segment (start 143.8 92.2) (end 142.6 92.2) (width 0.4) (layer B.Cu) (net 2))
 (segment (start 145 92.1) (end 143.9 92.1) (width 0.4) (layer F.Cu) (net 2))
 (segment (start 143.9 92.1) (end 143.8 92.2) (width 0.4) (layer F.Cu) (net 2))
 (segment (start 141.2 102.9) (end 141.2 102.0499) (width 0.4) (layer F.Cu) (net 2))
 (segment (start 141.2 102.0499) (end 140.8 101.6499) (width 0.4) (layer F.Cu) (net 2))
 (segment (start 140.8 101.6499) (end 140.8 98.8) (width 0.4) (layer F.Cu) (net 2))
 (segment (start 141.15 103.6012) (end 141.2 103.5512) (width 0.4) (layer F.Cu) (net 2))
 (segment (start 141.2 103.5512) (end 141.2 102.9) (width 0.4) (layer F.Cu) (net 2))
 (segment (start 141.15 105.251) (end 142.4505 105.251) (width 0.4) (layer F.Cu) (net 2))
 (segment (start 144.8 106.175) (end 143.3745 106.175) (width 0.4) (layer F.Cu) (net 2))
 (segment (start 143.3745 106.175) (end 142.4505 105.251) (width 0.4) (layer F.Cu) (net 2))
 (segment (start 141.55 96.9) (end 141.3 96.65) (width 0.4) (layer F.Cu) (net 2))
 (segment (start 141.3 96.65) (end 141.3 96.225) (width 0.4) (layer F.Cu) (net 2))
 (segment (start 141.3 97.575) (end 141.55 97.325) (width 0.4) (layer F.Cu) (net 2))
 (segment (start 141.55 97.325) (end 141.55 96.9) (width 0.4) (layer F.Cu) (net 2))
 (segment (start 138.8999 95.4) (end 138.8999 95.55) (width 0.4) (layer F.Cu) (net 2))
 (segment (start 141.3 94.875) (end 139.4249 94.875) (width 0.4) (layer F.Cu) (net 2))
 (segment (start 139.4249 94.875) (end 138.8999 95.4) (width 0.4) (layer F.Cu) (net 2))
 (segment (start 138.8999 95.4) (end 138 95.4) (width 0.4) (layer F.Cu) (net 2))
 (segment (start 141.55 95.55) (end 138.8999 95.55) (width 0.4) (layer F.Cu) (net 2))
 (segment (start 141.55 94.2) (end 141.3 94.45) (width 0.4) (layer F.Cu) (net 2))
 (segment (start 141.3 94.45) (end 141.3 94.875) (width 0.4) (layer F.Cu) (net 2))
 (segment (start 141.3 96.225) (end 141.55 95.975) (width 0.4) (layer F.Cu) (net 2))
 (segment (start 141.55 95.975) (end 141.55 95.55) (width 0.4) (layer F.Cu) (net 2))
 (segment (start 141.55 94.2) (end 141.3 93.95) (width 0.4) (layer F.Cu) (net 2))
 (segment (start 141.3 93.95) (end 141.3 93.525) (width 0.4) (layer F.Cu) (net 2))
 (segment (start 141.15 105.251) (end 141.15 103.6012) (width 0.4) (layer F.Cu) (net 2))
 (segment (start 132.4 95.4) (end 138 95.4) (width 0.4) (layer F.Cu) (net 2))
 (segment (start 153.45 108.9) (end 153.45 107.65) (width 0.4) (layer F.Cu) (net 10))
 (segment (start 153.45 107.65) (end 153.5 107.6) (width 0.4) (layer F.Cu) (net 10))
 (segment (start 146.4 97.6) (end 145.4 98.6) (width 0.4) (layer B.Cu) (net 1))
 (segment (start 145.4 98.6) (end 145.4 99.8) (width 0.4) (layer B.Cu) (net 1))
 (segment (start 146.4 96.4) (end 146.4 97.6) (width 0.4) (layer B.Cu) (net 1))
 (segment (start 146.4 95.2) (end 146.4 96.4) (width 0.4) (layer B.Cu) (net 1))
 (segment (start 145.1225 102.35) (end 145.4 102.0725) (width 0.4) (layer F.Cu) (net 1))
 (segment (start 145.4 102.0725) (end 145.4 99.8) (width 0.4) (layer F.Cu) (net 1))
 (segment (start 145.1225 102.35) (end 144.7749 102.35) (width 0.4) (layer F.Cu) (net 1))
 (segment (start 145.47 102.35) (end 145.1225 102.35) (width 0.4) (layer F.Cu) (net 1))
 (segment (start 144.8 104.875) (end 143.6749 104.875) (width 0.4) (layer F.Cu) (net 1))
 (segment (start 143.6749 104.875) (end 143.6749 103.45) (width 0.4) (layer F.Cu) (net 1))
 (segment (start 143.6749 103.45) (end 144.7749 102.35) (width 0.4) (layer F.Cu) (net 1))
 (segment (start 147.675 95.32) (end 146.52 95.32) (width 0.4) (layer F.Cu) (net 1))
 (segment (start 146.52 95.32) (end 146.4 95.2) (width 0.4) (layer F.Cu) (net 1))
 (segment (start 147.675 96.59) (end 146.59 96.59) (width 0.4) (layer F.Cu) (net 1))
 (segment (start 146.59 96.59) (end 146.4 96.4) (width 0.4) (layer F.Cu) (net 1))
 (segment (start 147.675 97.86) (end 146.66 97.86) (width 0.4) (layer F.Cu) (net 1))
 (segment (start 146.66 97.86) (end 146.4 97.6) (width 0.4) (layer F.Cu) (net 1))
 (segment (start 145 97.455) (end 146.255 97.455) (width 0.4) (layer F.Cu) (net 1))
 (segment (start 146.255 97.455) (end 146.4 97.6) (width 0.4) (layer F.Cu) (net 1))
 (segment (start 145 96.185) (end 146.185 96.185) (width 0.4) (layer F.Cu) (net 1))
 (segment (start 146.185 96.185) (end 146.4 96.4) (width 0.4) (layer F.Cu) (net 1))
 (segment (start 145 94.915) (end 146.115 94.915) (width 0.4) (layer F.Cu) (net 1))
 (segment (start 146.115 94.915) (end 146.4 95.2) (width 0.4) (layer F.Cu) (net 1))
 (segment (start 146.7 93.7) (end 145.055 93.7) (width 0.4) (layer F.Cu) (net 9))
 (segment (start 145.055 93.7) (end 145 93.645) (width 0.4) (layer F.Cu) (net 9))
 (segment (start 139.25 103.8) (end 139.25 103.35) (width 0.4) (layer F.Cu) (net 7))
 (segment (start 139.25 103.35) (end 139.7 102.9) (width 0.4) (layer F.Cu) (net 7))
 (segment (start 149.2 106.175) (end 147.475 106.175) (width 0.4) (layer F.Cu) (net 7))
 (segment (start 147.475 106.175) (end 146.4 107.25) (width 0.4) (layer F.Cu) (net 7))
 (segment (start 146.4 107.25) (end 139.8 107.25) (width 0.4) (layer F.Cu) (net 7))
 (segment (start 139.8 107.25) (end 139.25 106.7) (width 0.4) (layer F.Cu) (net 7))
 (segment (start 139.25 106.7) (end 139.25 103.8) (width 0.4) (layer F.Cu) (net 7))
 (segment (start 137.33 103.85) (end 139.2 103.85) (width 0.4) (layer F.Cu) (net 7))
 (segment (start 139.2 103.85) (end 139.25 103.8) (width 0.4) (layer F.Cu) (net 7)))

